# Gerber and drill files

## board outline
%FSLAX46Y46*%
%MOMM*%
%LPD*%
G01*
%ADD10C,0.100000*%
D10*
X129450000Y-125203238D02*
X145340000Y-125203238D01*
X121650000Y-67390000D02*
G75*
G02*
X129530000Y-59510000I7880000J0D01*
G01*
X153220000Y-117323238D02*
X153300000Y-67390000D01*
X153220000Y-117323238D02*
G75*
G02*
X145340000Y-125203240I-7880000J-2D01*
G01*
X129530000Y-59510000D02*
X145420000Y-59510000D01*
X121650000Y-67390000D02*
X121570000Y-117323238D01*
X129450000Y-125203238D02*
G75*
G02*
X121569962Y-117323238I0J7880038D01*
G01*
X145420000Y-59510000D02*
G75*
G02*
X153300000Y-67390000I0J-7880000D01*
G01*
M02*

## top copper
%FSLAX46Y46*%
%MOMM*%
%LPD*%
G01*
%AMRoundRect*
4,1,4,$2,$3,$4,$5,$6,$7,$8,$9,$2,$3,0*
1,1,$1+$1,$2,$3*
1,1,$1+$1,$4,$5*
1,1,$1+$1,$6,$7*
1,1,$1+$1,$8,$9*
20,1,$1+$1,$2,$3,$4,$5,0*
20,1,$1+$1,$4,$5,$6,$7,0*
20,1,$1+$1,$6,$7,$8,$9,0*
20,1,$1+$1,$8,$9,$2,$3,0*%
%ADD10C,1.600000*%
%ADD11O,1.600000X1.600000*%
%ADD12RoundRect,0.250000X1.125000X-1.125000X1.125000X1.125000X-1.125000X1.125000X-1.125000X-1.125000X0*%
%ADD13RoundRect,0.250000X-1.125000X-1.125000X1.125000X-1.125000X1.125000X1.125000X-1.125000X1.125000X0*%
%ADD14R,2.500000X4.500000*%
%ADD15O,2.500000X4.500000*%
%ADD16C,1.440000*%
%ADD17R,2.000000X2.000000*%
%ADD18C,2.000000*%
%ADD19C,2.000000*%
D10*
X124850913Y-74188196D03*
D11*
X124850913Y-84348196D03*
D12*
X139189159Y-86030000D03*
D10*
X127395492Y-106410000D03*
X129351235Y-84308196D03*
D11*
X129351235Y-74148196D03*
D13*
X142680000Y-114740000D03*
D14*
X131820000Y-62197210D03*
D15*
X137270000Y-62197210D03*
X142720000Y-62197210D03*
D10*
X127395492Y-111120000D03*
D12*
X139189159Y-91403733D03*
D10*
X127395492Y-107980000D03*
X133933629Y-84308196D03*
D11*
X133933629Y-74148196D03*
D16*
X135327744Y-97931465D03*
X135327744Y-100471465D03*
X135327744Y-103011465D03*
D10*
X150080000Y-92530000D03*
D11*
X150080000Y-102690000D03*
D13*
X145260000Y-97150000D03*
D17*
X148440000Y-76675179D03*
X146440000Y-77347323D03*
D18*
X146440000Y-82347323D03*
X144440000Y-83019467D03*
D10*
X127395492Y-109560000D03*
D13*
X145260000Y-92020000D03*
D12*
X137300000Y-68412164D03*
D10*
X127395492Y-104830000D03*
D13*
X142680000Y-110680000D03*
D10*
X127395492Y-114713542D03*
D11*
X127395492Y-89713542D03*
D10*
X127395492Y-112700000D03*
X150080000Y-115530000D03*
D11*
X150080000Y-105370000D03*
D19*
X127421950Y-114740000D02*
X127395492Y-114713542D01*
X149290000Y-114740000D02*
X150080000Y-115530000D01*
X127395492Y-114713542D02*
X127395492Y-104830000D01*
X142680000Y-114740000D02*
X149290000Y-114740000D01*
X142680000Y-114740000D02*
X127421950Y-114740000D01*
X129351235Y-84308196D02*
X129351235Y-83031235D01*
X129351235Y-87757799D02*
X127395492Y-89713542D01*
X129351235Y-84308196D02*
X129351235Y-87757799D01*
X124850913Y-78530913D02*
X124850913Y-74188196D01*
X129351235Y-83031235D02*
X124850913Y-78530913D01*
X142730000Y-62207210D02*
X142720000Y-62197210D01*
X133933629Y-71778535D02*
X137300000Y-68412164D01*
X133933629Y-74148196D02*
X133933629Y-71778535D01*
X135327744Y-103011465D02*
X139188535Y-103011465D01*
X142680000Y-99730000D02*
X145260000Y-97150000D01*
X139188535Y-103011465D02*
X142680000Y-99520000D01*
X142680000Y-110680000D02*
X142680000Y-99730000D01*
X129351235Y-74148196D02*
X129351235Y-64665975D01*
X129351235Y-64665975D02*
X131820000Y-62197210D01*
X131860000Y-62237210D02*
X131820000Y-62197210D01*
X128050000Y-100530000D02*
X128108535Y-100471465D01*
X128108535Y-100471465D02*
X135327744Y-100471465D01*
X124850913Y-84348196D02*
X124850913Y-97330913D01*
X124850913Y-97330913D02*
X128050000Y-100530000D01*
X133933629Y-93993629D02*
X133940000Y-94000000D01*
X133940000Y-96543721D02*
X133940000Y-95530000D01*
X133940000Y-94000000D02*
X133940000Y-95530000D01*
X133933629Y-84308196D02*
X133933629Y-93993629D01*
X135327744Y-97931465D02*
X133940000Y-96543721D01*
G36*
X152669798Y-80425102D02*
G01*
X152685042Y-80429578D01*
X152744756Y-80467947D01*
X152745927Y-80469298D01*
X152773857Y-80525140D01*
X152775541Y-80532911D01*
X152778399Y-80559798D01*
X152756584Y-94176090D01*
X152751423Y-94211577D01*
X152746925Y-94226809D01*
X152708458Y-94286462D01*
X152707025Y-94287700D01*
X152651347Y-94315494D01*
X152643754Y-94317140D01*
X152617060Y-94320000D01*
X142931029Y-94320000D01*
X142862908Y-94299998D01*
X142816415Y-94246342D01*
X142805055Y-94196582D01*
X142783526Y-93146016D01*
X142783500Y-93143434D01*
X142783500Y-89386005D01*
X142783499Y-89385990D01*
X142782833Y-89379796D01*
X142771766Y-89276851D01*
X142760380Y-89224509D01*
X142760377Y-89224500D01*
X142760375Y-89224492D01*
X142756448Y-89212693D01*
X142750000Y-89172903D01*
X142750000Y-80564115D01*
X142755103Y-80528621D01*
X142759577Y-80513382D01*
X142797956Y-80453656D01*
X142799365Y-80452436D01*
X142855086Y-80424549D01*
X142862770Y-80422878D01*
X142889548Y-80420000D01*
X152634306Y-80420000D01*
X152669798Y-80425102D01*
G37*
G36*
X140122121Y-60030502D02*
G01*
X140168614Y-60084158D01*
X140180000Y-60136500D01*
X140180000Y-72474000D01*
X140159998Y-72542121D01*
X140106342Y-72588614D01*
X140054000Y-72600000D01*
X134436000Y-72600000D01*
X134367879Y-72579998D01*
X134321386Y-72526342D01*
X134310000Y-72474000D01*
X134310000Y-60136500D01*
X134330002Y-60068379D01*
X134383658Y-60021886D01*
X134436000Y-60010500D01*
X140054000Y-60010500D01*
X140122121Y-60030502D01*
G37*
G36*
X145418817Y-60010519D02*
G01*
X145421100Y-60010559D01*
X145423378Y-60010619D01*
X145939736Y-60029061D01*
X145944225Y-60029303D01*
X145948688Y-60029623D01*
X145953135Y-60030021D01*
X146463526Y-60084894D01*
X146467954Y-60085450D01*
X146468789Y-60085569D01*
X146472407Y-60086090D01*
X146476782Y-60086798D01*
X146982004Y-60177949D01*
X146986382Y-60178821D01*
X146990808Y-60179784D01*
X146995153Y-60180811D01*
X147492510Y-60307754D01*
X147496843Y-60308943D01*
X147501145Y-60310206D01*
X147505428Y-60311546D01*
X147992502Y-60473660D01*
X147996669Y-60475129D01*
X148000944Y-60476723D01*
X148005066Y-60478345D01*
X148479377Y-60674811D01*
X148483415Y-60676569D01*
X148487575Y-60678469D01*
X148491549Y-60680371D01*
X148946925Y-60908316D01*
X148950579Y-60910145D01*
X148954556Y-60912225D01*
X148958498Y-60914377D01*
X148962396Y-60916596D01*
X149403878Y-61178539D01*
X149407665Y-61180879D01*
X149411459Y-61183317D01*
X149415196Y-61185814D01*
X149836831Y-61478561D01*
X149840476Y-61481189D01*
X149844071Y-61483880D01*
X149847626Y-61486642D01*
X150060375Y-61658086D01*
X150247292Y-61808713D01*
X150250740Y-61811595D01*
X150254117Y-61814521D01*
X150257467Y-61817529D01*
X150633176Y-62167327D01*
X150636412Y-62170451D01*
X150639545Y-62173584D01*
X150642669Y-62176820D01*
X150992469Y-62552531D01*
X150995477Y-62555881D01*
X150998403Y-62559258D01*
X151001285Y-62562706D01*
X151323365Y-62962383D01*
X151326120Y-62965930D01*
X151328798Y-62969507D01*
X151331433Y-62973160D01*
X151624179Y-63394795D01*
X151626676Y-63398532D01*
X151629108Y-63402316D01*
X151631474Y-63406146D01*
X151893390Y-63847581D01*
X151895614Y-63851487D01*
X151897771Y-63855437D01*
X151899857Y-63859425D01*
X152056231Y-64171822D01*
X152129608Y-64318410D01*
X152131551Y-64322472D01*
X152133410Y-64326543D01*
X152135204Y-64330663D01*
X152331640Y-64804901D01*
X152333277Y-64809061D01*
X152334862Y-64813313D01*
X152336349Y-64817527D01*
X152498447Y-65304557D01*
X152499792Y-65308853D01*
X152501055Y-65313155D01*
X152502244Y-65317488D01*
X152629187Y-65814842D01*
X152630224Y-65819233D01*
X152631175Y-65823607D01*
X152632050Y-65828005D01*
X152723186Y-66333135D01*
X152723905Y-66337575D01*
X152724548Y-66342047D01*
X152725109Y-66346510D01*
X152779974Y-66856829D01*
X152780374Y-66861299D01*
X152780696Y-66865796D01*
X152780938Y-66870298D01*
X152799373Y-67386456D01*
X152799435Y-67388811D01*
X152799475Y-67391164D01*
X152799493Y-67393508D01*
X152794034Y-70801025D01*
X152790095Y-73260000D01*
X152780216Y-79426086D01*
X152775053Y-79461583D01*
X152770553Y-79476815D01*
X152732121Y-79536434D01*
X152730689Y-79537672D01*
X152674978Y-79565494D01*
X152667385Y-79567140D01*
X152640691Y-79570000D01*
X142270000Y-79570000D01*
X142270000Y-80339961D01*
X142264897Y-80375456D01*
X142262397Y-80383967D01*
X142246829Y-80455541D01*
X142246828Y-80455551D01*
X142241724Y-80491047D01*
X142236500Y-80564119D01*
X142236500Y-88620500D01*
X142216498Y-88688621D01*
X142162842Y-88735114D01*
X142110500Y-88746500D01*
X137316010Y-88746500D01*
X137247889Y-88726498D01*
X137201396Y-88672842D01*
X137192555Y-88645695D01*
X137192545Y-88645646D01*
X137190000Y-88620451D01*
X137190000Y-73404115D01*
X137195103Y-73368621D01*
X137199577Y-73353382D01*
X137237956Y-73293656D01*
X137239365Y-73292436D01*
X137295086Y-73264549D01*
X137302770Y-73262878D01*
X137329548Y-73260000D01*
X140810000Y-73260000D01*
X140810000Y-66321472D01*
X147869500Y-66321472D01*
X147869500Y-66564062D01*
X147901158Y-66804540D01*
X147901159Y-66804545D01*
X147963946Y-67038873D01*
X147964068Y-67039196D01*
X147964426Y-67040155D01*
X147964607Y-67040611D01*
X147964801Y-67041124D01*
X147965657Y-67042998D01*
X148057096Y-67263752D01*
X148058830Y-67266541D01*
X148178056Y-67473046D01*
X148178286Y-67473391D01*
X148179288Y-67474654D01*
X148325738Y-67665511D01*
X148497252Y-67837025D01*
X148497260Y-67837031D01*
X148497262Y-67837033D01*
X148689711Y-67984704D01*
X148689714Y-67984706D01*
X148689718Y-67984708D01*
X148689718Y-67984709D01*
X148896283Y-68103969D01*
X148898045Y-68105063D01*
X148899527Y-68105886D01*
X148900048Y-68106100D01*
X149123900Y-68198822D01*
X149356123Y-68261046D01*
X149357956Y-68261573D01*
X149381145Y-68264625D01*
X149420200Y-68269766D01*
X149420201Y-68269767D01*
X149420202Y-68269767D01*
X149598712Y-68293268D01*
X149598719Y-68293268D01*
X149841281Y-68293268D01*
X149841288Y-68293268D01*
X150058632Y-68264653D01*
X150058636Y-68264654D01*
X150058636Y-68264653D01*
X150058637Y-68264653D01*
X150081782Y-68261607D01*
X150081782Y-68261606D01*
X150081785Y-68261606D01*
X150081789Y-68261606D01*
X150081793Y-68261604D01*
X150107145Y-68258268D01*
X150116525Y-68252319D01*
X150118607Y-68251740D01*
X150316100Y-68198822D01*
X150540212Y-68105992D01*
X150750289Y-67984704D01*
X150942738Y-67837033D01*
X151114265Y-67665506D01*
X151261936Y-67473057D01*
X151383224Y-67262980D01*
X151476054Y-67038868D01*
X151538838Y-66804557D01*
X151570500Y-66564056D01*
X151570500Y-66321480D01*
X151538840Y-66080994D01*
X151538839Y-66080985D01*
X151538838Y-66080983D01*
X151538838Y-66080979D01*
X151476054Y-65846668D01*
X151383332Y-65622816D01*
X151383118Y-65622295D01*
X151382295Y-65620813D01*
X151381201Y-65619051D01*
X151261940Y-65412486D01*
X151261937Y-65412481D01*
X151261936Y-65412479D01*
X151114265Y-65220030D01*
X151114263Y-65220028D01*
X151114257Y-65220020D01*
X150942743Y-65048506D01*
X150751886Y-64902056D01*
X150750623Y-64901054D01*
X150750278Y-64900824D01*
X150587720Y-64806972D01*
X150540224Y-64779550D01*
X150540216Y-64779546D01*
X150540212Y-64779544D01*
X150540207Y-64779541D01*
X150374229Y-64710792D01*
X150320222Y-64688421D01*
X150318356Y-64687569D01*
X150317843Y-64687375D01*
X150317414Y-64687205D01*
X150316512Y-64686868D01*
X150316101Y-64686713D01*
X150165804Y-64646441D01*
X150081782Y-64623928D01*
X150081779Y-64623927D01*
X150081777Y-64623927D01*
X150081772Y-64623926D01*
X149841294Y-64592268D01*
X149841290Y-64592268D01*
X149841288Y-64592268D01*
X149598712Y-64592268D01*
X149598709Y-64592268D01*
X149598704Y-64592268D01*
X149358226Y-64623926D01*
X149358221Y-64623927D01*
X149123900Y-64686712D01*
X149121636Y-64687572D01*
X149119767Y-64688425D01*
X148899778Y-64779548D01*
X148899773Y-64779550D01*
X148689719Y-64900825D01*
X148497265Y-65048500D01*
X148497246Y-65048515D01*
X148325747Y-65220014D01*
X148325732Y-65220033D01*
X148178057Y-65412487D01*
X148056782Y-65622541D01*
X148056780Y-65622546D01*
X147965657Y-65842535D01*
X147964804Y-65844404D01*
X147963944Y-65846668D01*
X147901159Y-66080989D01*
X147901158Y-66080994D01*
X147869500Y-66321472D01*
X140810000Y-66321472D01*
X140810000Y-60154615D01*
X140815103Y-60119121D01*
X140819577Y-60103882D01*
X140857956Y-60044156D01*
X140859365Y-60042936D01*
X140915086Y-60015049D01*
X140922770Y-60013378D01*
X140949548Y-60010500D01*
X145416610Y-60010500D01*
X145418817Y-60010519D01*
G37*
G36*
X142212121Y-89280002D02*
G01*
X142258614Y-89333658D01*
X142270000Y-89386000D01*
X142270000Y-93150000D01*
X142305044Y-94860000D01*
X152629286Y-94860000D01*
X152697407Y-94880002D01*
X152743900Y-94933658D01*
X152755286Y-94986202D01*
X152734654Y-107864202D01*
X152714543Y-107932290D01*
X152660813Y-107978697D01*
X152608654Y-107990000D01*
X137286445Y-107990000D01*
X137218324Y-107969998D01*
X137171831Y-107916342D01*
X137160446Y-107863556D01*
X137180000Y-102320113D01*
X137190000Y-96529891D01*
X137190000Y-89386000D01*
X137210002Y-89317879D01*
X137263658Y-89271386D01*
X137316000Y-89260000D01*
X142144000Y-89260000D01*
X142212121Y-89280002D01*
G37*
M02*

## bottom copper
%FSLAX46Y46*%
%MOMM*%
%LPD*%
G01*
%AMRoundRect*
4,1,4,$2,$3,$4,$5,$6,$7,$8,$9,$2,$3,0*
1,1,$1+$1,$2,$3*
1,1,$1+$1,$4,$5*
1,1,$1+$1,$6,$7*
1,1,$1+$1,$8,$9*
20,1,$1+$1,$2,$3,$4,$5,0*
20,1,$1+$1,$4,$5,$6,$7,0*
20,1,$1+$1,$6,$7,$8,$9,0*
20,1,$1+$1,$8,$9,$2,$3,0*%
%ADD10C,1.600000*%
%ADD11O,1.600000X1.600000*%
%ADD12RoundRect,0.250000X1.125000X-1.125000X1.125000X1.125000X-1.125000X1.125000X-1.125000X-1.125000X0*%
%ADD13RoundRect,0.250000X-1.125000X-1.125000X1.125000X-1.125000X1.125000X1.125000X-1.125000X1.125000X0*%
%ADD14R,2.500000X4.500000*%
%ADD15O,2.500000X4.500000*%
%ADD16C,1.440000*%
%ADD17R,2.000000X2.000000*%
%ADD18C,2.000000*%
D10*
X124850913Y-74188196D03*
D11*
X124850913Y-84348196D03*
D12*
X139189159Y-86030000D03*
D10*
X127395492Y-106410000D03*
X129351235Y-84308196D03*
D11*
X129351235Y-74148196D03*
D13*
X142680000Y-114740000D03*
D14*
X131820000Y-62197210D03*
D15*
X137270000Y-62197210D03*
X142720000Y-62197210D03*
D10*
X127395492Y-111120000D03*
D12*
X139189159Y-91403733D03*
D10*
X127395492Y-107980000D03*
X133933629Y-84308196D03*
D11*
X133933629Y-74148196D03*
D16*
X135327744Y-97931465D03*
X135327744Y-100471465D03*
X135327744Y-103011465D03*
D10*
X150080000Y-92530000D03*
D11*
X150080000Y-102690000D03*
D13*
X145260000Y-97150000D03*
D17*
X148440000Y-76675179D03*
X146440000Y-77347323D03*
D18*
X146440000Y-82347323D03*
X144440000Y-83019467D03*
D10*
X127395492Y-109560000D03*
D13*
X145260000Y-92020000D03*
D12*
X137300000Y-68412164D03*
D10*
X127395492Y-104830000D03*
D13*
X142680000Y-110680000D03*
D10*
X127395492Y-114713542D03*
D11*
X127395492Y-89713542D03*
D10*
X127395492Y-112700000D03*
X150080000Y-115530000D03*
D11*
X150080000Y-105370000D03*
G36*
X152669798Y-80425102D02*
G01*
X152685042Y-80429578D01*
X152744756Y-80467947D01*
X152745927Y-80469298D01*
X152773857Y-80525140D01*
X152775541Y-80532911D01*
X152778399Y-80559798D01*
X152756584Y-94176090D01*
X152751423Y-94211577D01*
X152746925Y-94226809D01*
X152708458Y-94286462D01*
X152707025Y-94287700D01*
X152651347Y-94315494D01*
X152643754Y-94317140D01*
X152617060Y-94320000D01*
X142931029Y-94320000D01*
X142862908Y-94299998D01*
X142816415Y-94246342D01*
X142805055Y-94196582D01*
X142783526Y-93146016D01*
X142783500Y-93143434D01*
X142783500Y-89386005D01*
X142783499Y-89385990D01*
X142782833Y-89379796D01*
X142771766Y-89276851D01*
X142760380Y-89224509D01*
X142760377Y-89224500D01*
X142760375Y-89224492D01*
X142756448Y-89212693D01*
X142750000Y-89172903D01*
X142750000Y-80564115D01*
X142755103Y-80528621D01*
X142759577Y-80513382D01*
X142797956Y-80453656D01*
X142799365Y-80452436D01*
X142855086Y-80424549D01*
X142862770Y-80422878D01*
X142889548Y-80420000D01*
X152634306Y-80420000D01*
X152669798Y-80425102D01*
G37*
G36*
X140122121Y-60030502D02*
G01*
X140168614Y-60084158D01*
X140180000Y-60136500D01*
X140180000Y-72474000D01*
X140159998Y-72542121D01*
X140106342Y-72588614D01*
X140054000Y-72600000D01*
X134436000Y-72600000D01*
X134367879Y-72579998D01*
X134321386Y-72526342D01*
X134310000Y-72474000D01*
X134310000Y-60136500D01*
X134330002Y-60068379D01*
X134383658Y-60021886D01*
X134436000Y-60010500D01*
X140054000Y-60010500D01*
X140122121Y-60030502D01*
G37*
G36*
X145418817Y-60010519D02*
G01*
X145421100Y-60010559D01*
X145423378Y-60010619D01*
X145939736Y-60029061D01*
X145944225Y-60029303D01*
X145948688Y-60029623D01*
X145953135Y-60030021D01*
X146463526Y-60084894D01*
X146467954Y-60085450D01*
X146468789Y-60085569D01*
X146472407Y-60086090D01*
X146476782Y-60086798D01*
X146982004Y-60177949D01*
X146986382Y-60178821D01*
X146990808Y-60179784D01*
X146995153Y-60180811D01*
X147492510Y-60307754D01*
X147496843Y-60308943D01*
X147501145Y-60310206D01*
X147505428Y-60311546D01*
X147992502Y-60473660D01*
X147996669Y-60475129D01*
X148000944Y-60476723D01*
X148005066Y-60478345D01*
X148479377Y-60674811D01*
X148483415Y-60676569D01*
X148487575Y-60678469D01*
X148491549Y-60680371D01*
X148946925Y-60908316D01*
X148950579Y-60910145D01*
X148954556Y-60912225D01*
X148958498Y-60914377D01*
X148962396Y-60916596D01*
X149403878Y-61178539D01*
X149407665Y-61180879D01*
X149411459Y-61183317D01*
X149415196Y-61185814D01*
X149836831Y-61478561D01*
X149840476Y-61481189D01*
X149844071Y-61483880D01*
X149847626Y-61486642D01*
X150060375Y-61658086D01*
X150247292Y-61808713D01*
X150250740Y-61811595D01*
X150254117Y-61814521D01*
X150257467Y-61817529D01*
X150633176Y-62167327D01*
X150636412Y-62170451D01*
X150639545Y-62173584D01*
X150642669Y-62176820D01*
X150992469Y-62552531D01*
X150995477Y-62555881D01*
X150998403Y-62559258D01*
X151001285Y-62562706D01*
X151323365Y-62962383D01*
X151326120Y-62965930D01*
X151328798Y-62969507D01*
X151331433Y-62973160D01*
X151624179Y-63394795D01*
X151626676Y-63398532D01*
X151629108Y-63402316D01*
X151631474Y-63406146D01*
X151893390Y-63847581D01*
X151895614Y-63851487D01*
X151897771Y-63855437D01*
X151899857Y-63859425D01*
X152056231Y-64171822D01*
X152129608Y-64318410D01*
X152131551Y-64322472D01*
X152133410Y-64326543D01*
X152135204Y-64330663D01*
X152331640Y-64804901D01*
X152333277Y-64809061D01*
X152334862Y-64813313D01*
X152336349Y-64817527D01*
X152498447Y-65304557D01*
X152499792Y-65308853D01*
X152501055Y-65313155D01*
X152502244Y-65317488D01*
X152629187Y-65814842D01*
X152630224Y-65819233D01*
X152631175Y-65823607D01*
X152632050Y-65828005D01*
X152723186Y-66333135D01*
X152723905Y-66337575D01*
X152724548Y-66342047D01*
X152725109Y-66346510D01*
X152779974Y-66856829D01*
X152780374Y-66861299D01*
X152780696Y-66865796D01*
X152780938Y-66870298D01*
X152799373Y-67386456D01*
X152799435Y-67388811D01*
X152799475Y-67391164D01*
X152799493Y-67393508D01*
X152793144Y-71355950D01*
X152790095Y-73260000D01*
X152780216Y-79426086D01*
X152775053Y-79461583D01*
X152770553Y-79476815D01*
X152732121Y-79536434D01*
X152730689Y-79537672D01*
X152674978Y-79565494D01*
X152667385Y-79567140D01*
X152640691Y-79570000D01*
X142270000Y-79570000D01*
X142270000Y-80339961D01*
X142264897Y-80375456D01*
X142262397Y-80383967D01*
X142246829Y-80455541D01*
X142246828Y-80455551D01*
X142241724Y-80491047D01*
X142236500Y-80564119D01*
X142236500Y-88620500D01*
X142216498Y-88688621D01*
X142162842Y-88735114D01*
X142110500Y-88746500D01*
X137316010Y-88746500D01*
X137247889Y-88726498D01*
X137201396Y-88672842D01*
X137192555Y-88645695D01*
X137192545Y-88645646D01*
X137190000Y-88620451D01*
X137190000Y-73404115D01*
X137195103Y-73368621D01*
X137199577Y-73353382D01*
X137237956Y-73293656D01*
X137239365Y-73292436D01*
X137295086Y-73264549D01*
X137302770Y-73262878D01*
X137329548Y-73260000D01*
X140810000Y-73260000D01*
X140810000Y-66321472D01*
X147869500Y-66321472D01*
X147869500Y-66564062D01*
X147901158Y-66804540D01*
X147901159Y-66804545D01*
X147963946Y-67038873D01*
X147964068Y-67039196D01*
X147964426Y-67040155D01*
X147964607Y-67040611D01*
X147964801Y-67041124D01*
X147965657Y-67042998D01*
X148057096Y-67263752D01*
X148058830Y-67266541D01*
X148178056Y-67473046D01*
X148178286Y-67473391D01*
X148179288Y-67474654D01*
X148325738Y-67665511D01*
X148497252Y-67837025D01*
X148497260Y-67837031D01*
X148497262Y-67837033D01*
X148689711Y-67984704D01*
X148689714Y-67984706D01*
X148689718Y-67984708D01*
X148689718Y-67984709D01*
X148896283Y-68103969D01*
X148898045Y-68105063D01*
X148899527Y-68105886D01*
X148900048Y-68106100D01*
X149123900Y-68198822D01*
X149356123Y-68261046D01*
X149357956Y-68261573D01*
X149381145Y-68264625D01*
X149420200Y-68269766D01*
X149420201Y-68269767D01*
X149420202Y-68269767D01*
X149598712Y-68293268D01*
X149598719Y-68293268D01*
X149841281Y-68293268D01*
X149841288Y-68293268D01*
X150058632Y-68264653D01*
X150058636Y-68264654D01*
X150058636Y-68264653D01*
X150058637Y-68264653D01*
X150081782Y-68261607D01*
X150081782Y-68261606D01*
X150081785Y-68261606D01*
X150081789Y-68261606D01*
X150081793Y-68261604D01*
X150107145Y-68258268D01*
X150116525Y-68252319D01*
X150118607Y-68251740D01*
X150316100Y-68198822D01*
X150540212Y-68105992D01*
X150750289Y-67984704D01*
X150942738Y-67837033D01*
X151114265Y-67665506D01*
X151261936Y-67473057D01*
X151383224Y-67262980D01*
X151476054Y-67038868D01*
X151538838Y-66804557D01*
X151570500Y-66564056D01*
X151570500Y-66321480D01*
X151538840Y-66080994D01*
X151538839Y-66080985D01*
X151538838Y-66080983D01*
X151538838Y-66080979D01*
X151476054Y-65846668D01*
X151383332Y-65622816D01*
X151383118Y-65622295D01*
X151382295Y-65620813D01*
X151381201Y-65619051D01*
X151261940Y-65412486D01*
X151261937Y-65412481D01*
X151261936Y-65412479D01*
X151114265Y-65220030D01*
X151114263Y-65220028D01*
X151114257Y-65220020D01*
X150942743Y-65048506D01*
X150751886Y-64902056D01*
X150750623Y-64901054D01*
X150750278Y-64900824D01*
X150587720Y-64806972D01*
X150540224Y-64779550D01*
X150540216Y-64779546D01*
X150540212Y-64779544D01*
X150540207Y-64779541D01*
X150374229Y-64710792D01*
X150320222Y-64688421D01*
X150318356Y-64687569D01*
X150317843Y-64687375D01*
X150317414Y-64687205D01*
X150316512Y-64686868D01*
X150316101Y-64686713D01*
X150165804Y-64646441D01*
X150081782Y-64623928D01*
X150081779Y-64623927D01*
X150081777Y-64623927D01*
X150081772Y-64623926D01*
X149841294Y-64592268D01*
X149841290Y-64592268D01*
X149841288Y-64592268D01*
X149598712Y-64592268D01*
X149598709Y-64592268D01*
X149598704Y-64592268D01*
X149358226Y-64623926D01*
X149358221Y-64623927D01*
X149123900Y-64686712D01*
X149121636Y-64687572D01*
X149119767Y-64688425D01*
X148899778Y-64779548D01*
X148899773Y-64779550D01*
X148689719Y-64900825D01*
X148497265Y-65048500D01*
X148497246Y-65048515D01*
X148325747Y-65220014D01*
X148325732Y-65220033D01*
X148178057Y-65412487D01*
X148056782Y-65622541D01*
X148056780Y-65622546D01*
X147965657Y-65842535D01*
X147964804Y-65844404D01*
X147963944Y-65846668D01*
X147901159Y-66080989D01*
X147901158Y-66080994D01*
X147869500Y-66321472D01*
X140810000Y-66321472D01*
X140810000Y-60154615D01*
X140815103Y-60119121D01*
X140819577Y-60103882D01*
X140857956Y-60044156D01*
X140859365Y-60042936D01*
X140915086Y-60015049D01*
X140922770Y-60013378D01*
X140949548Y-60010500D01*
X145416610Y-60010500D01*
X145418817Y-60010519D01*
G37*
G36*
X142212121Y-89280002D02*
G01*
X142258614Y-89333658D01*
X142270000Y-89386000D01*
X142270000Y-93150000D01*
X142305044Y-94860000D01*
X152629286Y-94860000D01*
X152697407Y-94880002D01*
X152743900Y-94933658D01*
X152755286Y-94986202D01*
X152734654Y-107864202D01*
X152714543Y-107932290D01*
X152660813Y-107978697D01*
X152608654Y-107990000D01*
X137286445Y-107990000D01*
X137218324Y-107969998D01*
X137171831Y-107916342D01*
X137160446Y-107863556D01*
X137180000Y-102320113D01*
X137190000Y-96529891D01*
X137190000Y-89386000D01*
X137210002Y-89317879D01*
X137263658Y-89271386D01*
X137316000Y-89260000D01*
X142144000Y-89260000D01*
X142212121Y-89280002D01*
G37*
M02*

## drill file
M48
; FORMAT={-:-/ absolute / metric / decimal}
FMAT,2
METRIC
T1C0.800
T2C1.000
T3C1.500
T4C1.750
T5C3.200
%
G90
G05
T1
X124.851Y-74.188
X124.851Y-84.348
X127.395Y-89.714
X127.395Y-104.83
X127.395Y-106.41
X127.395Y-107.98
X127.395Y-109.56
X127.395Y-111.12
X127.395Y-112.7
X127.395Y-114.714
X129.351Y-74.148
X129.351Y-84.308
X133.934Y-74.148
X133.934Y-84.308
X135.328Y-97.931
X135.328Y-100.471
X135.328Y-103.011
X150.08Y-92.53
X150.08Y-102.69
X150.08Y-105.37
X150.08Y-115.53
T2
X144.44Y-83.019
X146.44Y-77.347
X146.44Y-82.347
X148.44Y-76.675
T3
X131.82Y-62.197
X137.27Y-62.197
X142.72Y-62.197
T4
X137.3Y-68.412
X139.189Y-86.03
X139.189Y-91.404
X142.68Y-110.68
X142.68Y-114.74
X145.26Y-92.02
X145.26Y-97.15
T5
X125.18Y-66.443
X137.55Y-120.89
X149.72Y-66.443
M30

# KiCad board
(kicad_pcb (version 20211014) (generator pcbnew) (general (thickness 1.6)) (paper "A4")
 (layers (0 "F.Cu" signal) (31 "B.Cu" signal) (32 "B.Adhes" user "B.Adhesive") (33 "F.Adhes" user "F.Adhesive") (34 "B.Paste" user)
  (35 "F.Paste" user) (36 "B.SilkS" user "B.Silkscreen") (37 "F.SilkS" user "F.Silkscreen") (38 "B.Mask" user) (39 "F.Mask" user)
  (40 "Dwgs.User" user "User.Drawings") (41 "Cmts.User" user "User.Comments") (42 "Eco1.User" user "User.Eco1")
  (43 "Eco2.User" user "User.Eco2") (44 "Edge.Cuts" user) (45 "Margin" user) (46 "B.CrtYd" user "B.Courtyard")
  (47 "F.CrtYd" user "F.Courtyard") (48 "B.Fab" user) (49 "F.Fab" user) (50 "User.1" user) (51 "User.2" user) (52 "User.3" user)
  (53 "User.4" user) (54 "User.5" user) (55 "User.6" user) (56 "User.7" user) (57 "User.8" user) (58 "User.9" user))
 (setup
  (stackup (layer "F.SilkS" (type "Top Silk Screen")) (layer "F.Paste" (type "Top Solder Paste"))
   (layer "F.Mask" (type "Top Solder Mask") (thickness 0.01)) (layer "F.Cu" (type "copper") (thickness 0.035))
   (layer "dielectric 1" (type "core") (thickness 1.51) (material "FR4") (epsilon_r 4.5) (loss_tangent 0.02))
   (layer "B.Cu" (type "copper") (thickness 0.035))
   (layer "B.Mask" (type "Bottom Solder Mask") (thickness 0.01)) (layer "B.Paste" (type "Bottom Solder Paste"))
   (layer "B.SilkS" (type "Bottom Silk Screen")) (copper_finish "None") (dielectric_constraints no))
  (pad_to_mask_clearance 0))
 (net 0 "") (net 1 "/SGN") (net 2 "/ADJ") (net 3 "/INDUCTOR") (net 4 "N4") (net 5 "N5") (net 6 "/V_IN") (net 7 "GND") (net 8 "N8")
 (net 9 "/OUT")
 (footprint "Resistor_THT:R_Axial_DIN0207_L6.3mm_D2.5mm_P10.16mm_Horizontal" (layer "F.Cu") (at 124.850913 74.188196 -90)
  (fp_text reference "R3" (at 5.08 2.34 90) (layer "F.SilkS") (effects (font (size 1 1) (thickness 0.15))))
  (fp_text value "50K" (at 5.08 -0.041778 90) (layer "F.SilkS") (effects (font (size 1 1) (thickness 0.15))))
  (pad "1" thru_hole circle locked (at 0 0 270) (size 1.6 1.6) (drill 0.8) (layers *.Cu *.Mask) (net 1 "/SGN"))
  (pad "2" thru_hole oval locked (at 10.16 0 270) (size 1.6 1.6) (drill 0.8) (layers *.Cu *.Mask) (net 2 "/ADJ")))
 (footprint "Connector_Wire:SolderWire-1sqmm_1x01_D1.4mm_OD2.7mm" (layer "F.Cu") (at 139.189159 86.03 90)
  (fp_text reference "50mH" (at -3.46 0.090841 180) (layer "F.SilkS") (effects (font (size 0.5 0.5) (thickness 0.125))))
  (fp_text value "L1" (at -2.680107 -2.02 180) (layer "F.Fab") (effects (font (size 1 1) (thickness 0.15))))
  (pad "1" thru_hole roundrect locked (at 0 0 90) (size 2.75 2.75) (drill 1.75) (layers *.Cu *.Mask) (roundrect_rratio 0.09090909091)
   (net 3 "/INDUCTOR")))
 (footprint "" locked (layer "F.Cu") (at 127.395492 106.41)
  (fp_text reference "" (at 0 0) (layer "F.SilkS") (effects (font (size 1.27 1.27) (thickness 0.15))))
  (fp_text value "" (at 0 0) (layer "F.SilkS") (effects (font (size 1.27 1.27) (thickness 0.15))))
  (pad "1" thru_hole circle locked (at 0 0 90) (size 1.6 1.6) (drill 0.8) (layers *.Cu *.Mask) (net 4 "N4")))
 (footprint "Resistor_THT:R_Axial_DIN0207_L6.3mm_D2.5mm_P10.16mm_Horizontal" (layer "F.Cu") (at 129.351235 84.308196 90)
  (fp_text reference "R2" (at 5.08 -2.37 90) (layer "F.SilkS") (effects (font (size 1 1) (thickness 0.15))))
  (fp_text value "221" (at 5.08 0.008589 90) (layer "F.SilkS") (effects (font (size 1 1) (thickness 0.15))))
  (pad "1" thru_hole circle locked (at 0 0 90) (size 1.6 1.6) (drill 0.8) (layers *.Cu *.Mask) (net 1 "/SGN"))
  (pad "2" thru_hole oval locked (at 10.16 0 90) (size 1.6 1.6) (drill 0.8) (layers *.Cu *.Mask) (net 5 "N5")))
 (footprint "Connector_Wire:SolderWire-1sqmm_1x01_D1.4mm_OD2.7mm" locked (layer "F.Cu") (at 142.68 114.74)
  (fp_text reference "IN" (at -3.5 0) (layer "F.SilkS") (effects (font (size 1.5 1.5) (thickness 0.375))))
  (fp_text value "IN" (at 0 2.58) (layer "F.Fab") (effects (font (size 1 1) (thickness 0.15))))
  (pad "1" thru_hole roundrect locked (at 0 0) (size 2.75 2.75) (drill 1.75) (layers *.Cu *.Mask) (roundrect_rratio 0.09090909091)
   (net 4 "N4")))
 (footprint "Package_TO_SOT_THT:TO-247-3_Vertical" (layer "F.Cu") (at 131.82 62.19721)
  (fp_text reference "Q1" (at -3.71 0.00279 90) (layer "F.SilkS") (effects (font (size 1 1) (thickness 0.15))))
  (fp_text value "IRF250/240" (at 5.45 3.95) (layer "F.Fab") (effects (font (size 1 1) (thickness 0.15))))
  (pad "1" thru_hole rect locked (at 0 0) (size 2.5 4.5) (drill 1.5) (layers *.Cu *.Mask) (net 5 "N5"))
  (pad "2" thru_hole oval locked (at 5.45 0) (size 2.5 4.5) (drill 1.5) (layers *.Cu *.Mask) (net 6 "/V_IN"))
  (pad "3" thru_hole oval locked (at 10.9 0) (size 2.5 4.5) (drill 1.5) (layers *.Cu *.Mask) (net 3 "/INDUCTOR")))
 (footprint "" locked (layer "F.Cu") (at 127.395492 111.12)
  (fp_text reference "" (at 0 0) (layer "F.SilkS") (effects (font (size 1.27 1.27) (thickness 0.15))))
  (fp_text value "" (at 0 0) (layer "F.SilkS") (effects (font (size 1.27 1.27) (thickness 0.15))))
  (pad "1" thru_hole circle locked (at 0 0 90) (size 1.6 1.6) (drill 0.8) (layers *.Cu *.Mask) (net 4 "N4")))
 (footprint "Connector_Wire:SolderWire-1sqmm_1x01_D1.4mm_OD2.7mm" (layer "F.Cu") (at 139.189159 91.403733 90)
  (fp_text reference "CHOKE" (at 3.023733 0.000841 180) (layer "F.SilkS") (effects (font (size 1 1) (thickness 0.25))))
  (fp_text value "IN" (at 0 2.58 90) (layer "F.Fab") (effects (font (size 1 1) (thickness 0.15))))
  (pad "1" thru_hole roundrect locked (at 0 0 90) (size 2.75 2.75) (drill 1.75) (layers *.Cu *.Mask) (roundrect_rratio 0.09090909091)
   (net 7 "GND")))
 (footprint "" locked (layer "F.Cu") (at 127.395492 107.98)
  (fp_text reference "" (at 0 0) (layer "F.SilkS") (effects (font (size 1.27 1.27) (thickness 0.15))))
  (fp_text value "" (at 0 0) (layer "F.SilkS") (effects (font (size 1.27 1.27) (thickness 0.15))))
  (pad "1" thru_hole circle locked (at 0 0 90) (size 1.6 1.6) (drill 0.8) (layers *.Cu *.Mask) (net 4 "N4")))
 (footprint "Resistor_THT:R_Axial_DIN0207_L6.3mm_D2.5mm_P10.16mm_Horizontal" (layer "F.Cu") (at 133.933629 84.308196 90)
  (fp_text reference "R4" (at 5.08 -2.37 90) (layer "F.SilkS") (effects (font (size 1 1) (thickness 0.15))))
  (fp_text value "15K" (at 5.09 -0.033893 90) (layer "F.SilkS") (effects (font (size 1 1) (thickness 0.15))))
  (pad "1" thru_hole circle locked (at 0 0 90) (size 1.6 1.6) (drill 0.8) (layers *.Cu *.Mask) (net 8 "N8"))
  (pad "2" thru_hole oval locked (at 10.16 0 90) (size 1.6 1.6) (drill 0.8) (layers *.Cu *.Mask) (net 6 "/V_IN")))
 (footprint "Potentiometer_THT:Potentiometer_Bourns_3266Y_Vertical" (layer "F.Cu") (at 135.327744 97.931465 90)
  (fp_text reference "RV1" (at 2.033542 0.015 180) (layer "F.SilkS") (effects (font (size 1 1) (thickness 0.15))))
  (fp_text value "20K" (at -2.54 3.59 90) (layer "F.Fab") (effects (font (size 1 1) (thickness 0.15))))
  (pad "1" thru_hole circle locked (at 0 0 90) (size 1.44 1.44) (drill 0.8) (layers *.Cu *.Mask) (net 8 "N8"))
  (pad "2" thru_hole circle locked (at -2.54 0 90) (size 1.44 1.44) (drill 0.8) (layers *.Cu *.Mask) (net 2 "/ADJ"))
  (pad "3" thru_hole circle locked (at -5.08 0 90) (size 1.44 1.44) (drill 0.8) (layers *.Cu *.Mask) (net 7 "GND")))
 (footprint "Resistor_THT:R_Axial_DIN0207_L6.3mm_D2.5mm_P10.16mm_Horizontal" (layer "F.Cu") (at 150.08 92.53 -90)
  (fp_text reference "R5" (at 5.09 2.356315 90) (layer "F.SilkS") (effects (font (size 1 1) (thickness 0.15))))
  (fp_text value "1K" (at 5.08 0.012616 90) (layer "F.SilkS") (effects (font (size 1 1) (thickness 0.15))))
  (pad "1" thru_hole circle locked (at 0 0 270) (size 1.6 1.6) (drill 0.8) (layers *.Cu *.Mask) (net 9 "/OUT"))
  (pad "2" thru_hole oval locked (at 10.16 0 270) (size 1.6 1.6) (drill 0.8) (layers *.Cu *.Mask) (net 7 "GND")))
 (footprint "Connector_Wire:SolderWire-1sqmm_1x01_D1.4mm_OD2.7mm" (layer "F.Cu") (at 145.26 97.15)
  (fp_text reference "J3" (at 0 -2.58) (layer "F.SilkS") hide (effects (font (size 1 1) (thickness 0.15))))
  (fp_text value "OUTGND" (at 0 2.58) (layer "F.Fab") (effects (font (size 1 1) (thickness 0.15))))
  (pad "1" thru_hole roundrect locked (at 0 0) (size 2.75 2.75) (drill 1.75) (layers *.Cu *.Mask) (roundrect_rratio 0.09090909091)
   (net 7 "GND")))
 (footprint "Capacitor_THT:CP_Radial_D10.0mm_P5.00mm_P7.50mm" (layer "F.Cu") (at 146.44 77.347323 -90)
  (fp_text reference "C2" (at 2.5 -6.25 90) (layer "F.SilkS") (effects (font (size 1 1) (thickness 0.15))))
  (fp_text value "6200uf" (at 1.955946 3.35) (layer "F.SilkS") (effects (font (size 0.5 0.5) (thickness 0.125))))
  (pad "1" thru_hole rect locked (at -0.672144 -2 270) (size 2 2) (drill 1) (layers *.Cu *.Mask) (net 3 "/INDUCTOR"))
  (pad "1" thru_hole rect locked (at 0 0 270) (size 2 2) (drill 1) (layers *.Cu *.Mask) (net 3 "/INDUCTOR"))
  (pad "2" thru_hole circle locked (at 5 0 270) (size 2 2) (drill 1) (layers *.Cu *.Mask) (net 9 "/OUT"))
  (pad "2" thru_hole circle locked (at 5.672144 2 270) (size 2 2) (drill 1) (layers *.Cu *.Mask) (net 9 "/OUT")))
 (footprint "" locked (layer "F.Cu") (at 127.395492 109.56)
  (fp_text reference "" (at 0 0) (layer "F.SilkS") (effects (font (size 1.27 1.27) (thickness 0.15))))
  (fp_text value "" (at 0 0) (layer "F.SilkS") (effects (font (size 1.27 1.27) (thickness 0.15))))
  (pad "1" thru_hole circle locked (at 0 0 90) (size 1.6 1.6) (drill 0.8) (layers *.Cu *.Mask) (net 4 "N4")))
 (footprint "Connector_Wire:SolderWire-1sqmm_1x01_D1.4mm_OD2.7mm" (layer "F.Cu") (at 145.26 92.02)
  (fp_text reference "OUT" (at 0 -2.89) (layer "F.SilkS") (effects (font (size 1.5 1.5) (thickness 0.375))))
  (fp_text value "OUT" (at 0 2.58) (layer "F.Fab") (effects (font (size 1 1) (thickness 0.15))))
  (pad "1" thru_hole roundrect locked (at 0 0) (size 2.75 2.75) (drill 1.75) (layers *.Cu *.Mask) (roundrect_rratio 0.09090909091)
   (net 9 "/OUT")))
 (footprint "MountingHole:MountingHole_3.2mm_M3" (layer "F.Cu") (at 125.18 66.442768)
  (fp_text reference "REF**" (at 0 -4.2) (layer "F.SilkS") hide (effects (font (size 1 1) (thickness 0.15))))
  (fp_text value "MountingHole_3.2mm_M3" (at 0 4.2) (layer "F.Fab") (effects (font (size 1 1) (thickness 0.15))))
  (pad "" np_thru_hole circle locked (at 0 0) (size 3.2 3.2) (drill 3.2) (layers *.Cu *.Mask)))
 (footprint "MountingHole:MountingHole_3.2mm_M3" (layer "F.Cu") (at 137.55 120.89)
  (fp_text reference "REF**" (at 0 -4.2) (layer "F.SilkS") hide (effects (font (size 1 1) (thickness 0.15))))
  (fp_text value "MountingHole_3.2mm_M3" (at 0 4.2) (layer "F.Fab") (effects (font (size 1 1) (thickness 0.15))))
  (pad "" np_thru_hole circle locked (at 0 0) (size 3.2 3.2) (drill 3.2) (layers *.Cu *.Mask)))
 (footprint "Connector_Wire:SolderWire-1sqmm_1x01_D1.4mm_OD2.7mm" (layer "F.Cu") (at 137.3 68.412164 90)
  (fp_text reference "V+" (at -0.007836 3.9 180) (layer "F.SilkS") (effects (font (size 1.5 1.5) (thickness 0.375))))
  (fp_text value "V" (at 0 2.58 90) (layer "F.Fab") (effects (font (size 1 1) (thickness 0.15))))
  (pad "1" thru_hole roundrect locked (at 0 0 90) (size 2.75 2.75) (drill 1.75) (layers *.Cu *.Mask) (roundrect_rratio 0.09090909091)
   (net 6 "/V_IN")))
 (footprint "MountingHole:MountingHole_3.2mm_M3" (layer "F.Cu") (at 149.72 66.442768)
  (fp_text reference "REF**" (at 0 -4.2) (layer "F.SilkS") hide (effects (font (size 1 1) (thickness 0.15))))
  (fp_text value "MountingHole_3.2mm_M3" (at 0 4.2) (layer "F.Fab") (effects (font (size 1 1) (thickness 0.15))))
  (pad "" np_thru_hole circle locked (at 0 0) (size 3.2 3.2) (drill 3.2) (layers *.Cu *.Mask)))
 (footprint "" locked (layer "F.Cu") (at 127.395492 104.83)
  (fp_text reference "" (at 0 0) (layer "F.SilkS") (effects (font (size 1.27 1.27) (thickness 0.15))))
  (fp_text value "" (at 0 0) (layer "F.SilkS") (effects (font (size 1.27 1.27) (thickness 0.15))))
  (pad "1" thru_hole circle locked (at 0 0 90) (size 1.6 1.6) (drill 0.8) (layers *.Cu *.Mask) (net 4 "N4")))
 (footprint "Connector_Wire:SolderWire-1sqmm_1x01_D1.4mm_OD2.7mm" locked (layer "F.Cu") (at 142.68 110.68)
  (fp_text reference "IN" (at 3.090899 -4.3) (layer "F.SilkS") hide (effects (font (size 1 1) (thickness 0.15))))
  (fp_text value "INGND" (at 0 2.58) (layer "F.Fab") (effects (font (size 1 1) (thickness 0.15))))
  (pad "1" thru_hole roundrect locked (at 0 0) (size 2.75 2.75) (drill 1.75) (layers *.Cu *.Mask) (roundrect_rratio 0.09090909091)
   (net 7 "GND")))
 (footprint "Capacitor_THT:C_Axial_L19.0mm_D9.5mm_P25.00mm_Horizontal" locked (layer "F.Cu") (at 127.395492 114.713542 90)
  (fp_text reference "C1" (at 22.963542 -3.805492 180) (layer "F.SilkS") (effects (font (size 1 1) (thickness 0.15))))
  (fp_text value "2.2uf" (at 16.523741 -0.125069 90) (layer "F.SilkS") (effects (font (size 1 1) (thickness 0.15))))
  (pad "1" thru_hole circle locked (at 0 0 90) (size 1.6 1.6) (drill 0.8) (layers *.Cu *.Mask) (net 4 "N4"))
  (pad "2" thru_hole oval locked (at 25 0 90) (size 1.6 1.6) (drill 0.8) (layers *.Cu *.Mask) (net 1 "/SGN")))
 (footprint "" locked (layer "F.Cu") (at 127.395492 112.7)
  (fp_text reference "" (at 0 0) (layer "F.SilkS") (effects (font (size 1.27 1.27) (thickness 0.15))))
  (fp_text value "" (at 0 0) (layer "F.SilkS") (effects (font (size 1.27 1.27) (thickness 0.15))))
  (pad "1" thru_hole circle locked (at 0 0 90) (size 1.6 1.6) (drill 0.8) (layers *.Cu *.Mask) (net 4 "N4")))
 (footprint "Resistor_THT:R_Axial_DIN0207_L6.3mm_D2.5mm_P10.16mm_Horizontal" (layer "F.Cu") (at 150.08 115.53 90)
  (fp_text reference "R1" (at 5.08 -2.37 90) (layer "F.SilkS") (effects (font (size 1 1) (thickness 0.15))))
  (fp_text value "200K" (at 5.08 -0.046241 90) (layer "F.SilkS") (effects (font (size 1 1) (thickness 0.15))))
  (pad "1" thru_hole circle locked (at 0 0 90) (size 1.6 1.6) (drill 0.8) (layers *.Cu *.Mask) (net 4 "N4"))
  (pad "2" thru_hole oval locked (at 10.16 0 90) (size 1.6 1.6) (drill 0.8) (layers *.Cu *.Mask) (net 7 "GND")))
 (gr_line locked (start 129.45 125.203238) (end 145.34 125.203238) (layer "Edge.Cuts") (width 0.1))
 (gr_arc locked (start 121.65 67.39) (mid 123.957999 61.817999) (end 129.53 59.51) (layer "Edge.Cuts") (width 0.1))
 (gr_line (start 153.22 117.323238) (end 153.3 67.39) (layer "Edge.Cuts") (width 0.1))
 (gr_arc locked (start 153.22 117.323238) (mid 150.912001 122.895239) (end 145.34 125.203238) (layer "Edge.Cuts") (width 0.1))
 (gr_line locked (start 129.53 59.51) (end 145.42 59.51) (layer "Edge.Cuts") (width 0.1))
 (gr_line (start 121.65 67.39) (end 121.57 117.323238) (layer "Edge.Cuts") (width 0.1))
 (gr_arc locked (start 129.45 125.203238) (mid 123.877999 122.895239) (end 121.57 117.323238) (layer "Edge.Cuts") (width 0.1))
 (gr_arc locked (start 145.42 59.51) (mid 150.992001 61.817999) (end 153.3 67.39) (layer "Edge.Cuts") (width 0.1))
 (segment (start 127.42195 114.74) (end 127.395492 114.713542) (width 2) (layer "F.Cu") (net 4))
 (segment (start 149.29 114.74) (end 150.08 115.53) (width 2) (layer "F.Cu") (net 4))
 (segment locked (start 127.395492 114.713542) (end 127.395492 104.83) (width 2) (layer "F.Cu") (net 4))
 (segment (start 142.68 114.74) (end 149.29 114.74) (width 2) (layer "F.Cu") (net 4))
 (segment (start 142.68 114.74) (end 127.42195 114.74) (width 2) (layer "F.Cu") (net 4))
 (segment (start 129.351235 84.308196) (end 129.351235 83.031235) (width 2) (layer "F.Cu") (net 1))
 (segment (start 129.351235 87.757799) (end 127.395492 89.713542) (width 2) (layer "F.Cu") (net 1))
 (segment (start 129.351235 84.308196) (end 129.351235 87.757799) (width 2) (layer "F.Cu") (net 1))
 (segment (start 124.850913 78.530913) (end 124.850913 74.188196) (width 2) (layer "F.Cu") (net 1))
 (segment (start 129.351235 83.031235) (end 124.850913 78.530913) (width 2) (layer "F.Cu") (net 1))
 (segment (start 142.73 62.20721) (end 142.72 62.19721) (width 2) (layer "F.Cu") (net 3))
 (segment (start 133.933629 71.778535) (end 137.3 68.412164) (width 2) (layer "F.Cu") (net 6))
 (segment (start 133.933629 74.148196) (end 133.933629 71.778535) (width 2) (layer "F.Cu") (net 6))
 (segment (start 135.327744 103.011465) (end 139.188535 103.011465) (width 2) (layer "F.Cu") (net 7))
 (segment (start 142.68 99.73) (end 145.26 97.15) (width 2) (layer "F.Cu") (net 7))
 (segment (start 139.188535 103.011465) (end 142.68 99.52) (width 2) (layer "F.Cu") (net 7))
 (segment (start 142.68 110.68) (end 142.68 99.73) (width 2) (layer "F.Cu") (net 7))
 (segment (start 129.351235 74.148196) (end 129.351235 64.665975) (width 2) (layer "F.Cu") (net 5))
 (segment (start 129.351235 64.665975) (end 131.82 62.19721) (width 2) (layer "F.Cu") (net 5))
 (segment (start 131.86 62.23721) (end 131.82 62.19721) (width 2) (layer "F.Cu") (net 5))
 (segment (start 128.05 100.53) (end 128.108535 100.471465) (width 2) (layer "F.Cu") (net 2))
 (segment (start 128.108535 100.471465) (end 135.327744 100.471465) (width 2) (layer "F.Cu") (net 2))
 (segment (start 124.850913 84.348196) (end 124.850913 97.330913) (width 2) (layer "F.Cu") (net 2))
 (segment (start 124.850913 97.330913) (end 128.05 100.53) (width 2) (layer "F.Cu") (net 2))
 (segment (start 133.933629 93.993629) (end 133.94 94) (width 2) (layer "F.Cu") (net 8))
 (segment (start 133.94 96.543721) (end 133.94 95.53) (width 2) (layer "F.Cu") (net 8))
 (segment (start 133.94 94) (end 133.94 95.53) (width 2) (layer "F.Cu") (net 8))
 (segment (start 133.933629 84.308196) (end 133.933629 93.993629) (width 2) (layer "F.Cu") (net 8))
 (segment (start 135.327744 97.931465) (end 133.94 96.543721) (width 2) (layer "F.Cu") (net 8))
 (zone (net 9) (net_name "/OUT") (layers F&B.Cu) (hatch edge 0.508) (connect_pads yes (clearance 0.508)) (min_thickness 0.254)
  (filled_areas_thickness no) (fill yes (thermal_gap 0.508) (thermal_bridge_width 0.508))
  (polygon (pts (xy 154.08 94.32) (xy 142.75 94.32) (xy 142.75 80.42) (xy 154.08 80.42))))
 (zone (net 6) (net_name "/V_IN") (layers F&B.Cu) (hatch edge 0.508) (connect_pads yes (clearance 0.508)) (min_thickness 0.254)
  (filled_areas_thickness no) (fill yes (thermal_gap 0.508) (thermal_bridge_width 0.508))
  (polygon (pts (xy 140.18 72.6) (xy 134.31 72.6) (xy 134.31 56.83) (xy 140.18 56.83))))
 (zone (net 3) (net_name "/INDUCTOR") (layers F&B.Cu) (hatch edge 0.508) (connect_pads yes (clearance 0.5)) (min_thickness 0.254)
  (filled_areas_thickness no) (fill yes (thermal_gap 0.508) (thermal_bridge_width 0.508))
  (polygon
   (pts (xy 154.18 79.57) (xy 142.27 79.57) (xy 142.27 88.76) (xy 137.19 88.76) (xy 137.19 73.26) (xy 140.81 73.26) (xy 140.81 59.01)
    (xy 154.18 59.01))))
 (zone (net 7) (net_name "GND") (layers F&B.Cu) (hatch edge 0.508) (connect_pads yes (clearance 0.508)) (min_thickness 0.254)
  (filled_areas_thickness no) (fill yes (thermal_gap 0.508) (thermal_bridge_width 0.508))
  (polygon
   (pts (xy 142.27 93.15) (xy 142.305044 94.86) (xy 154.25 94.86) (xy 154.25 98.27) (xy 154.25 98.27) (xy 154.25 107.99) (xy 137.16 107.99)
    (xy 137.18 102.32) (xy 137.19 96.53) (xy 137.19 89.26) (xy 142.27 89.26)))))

